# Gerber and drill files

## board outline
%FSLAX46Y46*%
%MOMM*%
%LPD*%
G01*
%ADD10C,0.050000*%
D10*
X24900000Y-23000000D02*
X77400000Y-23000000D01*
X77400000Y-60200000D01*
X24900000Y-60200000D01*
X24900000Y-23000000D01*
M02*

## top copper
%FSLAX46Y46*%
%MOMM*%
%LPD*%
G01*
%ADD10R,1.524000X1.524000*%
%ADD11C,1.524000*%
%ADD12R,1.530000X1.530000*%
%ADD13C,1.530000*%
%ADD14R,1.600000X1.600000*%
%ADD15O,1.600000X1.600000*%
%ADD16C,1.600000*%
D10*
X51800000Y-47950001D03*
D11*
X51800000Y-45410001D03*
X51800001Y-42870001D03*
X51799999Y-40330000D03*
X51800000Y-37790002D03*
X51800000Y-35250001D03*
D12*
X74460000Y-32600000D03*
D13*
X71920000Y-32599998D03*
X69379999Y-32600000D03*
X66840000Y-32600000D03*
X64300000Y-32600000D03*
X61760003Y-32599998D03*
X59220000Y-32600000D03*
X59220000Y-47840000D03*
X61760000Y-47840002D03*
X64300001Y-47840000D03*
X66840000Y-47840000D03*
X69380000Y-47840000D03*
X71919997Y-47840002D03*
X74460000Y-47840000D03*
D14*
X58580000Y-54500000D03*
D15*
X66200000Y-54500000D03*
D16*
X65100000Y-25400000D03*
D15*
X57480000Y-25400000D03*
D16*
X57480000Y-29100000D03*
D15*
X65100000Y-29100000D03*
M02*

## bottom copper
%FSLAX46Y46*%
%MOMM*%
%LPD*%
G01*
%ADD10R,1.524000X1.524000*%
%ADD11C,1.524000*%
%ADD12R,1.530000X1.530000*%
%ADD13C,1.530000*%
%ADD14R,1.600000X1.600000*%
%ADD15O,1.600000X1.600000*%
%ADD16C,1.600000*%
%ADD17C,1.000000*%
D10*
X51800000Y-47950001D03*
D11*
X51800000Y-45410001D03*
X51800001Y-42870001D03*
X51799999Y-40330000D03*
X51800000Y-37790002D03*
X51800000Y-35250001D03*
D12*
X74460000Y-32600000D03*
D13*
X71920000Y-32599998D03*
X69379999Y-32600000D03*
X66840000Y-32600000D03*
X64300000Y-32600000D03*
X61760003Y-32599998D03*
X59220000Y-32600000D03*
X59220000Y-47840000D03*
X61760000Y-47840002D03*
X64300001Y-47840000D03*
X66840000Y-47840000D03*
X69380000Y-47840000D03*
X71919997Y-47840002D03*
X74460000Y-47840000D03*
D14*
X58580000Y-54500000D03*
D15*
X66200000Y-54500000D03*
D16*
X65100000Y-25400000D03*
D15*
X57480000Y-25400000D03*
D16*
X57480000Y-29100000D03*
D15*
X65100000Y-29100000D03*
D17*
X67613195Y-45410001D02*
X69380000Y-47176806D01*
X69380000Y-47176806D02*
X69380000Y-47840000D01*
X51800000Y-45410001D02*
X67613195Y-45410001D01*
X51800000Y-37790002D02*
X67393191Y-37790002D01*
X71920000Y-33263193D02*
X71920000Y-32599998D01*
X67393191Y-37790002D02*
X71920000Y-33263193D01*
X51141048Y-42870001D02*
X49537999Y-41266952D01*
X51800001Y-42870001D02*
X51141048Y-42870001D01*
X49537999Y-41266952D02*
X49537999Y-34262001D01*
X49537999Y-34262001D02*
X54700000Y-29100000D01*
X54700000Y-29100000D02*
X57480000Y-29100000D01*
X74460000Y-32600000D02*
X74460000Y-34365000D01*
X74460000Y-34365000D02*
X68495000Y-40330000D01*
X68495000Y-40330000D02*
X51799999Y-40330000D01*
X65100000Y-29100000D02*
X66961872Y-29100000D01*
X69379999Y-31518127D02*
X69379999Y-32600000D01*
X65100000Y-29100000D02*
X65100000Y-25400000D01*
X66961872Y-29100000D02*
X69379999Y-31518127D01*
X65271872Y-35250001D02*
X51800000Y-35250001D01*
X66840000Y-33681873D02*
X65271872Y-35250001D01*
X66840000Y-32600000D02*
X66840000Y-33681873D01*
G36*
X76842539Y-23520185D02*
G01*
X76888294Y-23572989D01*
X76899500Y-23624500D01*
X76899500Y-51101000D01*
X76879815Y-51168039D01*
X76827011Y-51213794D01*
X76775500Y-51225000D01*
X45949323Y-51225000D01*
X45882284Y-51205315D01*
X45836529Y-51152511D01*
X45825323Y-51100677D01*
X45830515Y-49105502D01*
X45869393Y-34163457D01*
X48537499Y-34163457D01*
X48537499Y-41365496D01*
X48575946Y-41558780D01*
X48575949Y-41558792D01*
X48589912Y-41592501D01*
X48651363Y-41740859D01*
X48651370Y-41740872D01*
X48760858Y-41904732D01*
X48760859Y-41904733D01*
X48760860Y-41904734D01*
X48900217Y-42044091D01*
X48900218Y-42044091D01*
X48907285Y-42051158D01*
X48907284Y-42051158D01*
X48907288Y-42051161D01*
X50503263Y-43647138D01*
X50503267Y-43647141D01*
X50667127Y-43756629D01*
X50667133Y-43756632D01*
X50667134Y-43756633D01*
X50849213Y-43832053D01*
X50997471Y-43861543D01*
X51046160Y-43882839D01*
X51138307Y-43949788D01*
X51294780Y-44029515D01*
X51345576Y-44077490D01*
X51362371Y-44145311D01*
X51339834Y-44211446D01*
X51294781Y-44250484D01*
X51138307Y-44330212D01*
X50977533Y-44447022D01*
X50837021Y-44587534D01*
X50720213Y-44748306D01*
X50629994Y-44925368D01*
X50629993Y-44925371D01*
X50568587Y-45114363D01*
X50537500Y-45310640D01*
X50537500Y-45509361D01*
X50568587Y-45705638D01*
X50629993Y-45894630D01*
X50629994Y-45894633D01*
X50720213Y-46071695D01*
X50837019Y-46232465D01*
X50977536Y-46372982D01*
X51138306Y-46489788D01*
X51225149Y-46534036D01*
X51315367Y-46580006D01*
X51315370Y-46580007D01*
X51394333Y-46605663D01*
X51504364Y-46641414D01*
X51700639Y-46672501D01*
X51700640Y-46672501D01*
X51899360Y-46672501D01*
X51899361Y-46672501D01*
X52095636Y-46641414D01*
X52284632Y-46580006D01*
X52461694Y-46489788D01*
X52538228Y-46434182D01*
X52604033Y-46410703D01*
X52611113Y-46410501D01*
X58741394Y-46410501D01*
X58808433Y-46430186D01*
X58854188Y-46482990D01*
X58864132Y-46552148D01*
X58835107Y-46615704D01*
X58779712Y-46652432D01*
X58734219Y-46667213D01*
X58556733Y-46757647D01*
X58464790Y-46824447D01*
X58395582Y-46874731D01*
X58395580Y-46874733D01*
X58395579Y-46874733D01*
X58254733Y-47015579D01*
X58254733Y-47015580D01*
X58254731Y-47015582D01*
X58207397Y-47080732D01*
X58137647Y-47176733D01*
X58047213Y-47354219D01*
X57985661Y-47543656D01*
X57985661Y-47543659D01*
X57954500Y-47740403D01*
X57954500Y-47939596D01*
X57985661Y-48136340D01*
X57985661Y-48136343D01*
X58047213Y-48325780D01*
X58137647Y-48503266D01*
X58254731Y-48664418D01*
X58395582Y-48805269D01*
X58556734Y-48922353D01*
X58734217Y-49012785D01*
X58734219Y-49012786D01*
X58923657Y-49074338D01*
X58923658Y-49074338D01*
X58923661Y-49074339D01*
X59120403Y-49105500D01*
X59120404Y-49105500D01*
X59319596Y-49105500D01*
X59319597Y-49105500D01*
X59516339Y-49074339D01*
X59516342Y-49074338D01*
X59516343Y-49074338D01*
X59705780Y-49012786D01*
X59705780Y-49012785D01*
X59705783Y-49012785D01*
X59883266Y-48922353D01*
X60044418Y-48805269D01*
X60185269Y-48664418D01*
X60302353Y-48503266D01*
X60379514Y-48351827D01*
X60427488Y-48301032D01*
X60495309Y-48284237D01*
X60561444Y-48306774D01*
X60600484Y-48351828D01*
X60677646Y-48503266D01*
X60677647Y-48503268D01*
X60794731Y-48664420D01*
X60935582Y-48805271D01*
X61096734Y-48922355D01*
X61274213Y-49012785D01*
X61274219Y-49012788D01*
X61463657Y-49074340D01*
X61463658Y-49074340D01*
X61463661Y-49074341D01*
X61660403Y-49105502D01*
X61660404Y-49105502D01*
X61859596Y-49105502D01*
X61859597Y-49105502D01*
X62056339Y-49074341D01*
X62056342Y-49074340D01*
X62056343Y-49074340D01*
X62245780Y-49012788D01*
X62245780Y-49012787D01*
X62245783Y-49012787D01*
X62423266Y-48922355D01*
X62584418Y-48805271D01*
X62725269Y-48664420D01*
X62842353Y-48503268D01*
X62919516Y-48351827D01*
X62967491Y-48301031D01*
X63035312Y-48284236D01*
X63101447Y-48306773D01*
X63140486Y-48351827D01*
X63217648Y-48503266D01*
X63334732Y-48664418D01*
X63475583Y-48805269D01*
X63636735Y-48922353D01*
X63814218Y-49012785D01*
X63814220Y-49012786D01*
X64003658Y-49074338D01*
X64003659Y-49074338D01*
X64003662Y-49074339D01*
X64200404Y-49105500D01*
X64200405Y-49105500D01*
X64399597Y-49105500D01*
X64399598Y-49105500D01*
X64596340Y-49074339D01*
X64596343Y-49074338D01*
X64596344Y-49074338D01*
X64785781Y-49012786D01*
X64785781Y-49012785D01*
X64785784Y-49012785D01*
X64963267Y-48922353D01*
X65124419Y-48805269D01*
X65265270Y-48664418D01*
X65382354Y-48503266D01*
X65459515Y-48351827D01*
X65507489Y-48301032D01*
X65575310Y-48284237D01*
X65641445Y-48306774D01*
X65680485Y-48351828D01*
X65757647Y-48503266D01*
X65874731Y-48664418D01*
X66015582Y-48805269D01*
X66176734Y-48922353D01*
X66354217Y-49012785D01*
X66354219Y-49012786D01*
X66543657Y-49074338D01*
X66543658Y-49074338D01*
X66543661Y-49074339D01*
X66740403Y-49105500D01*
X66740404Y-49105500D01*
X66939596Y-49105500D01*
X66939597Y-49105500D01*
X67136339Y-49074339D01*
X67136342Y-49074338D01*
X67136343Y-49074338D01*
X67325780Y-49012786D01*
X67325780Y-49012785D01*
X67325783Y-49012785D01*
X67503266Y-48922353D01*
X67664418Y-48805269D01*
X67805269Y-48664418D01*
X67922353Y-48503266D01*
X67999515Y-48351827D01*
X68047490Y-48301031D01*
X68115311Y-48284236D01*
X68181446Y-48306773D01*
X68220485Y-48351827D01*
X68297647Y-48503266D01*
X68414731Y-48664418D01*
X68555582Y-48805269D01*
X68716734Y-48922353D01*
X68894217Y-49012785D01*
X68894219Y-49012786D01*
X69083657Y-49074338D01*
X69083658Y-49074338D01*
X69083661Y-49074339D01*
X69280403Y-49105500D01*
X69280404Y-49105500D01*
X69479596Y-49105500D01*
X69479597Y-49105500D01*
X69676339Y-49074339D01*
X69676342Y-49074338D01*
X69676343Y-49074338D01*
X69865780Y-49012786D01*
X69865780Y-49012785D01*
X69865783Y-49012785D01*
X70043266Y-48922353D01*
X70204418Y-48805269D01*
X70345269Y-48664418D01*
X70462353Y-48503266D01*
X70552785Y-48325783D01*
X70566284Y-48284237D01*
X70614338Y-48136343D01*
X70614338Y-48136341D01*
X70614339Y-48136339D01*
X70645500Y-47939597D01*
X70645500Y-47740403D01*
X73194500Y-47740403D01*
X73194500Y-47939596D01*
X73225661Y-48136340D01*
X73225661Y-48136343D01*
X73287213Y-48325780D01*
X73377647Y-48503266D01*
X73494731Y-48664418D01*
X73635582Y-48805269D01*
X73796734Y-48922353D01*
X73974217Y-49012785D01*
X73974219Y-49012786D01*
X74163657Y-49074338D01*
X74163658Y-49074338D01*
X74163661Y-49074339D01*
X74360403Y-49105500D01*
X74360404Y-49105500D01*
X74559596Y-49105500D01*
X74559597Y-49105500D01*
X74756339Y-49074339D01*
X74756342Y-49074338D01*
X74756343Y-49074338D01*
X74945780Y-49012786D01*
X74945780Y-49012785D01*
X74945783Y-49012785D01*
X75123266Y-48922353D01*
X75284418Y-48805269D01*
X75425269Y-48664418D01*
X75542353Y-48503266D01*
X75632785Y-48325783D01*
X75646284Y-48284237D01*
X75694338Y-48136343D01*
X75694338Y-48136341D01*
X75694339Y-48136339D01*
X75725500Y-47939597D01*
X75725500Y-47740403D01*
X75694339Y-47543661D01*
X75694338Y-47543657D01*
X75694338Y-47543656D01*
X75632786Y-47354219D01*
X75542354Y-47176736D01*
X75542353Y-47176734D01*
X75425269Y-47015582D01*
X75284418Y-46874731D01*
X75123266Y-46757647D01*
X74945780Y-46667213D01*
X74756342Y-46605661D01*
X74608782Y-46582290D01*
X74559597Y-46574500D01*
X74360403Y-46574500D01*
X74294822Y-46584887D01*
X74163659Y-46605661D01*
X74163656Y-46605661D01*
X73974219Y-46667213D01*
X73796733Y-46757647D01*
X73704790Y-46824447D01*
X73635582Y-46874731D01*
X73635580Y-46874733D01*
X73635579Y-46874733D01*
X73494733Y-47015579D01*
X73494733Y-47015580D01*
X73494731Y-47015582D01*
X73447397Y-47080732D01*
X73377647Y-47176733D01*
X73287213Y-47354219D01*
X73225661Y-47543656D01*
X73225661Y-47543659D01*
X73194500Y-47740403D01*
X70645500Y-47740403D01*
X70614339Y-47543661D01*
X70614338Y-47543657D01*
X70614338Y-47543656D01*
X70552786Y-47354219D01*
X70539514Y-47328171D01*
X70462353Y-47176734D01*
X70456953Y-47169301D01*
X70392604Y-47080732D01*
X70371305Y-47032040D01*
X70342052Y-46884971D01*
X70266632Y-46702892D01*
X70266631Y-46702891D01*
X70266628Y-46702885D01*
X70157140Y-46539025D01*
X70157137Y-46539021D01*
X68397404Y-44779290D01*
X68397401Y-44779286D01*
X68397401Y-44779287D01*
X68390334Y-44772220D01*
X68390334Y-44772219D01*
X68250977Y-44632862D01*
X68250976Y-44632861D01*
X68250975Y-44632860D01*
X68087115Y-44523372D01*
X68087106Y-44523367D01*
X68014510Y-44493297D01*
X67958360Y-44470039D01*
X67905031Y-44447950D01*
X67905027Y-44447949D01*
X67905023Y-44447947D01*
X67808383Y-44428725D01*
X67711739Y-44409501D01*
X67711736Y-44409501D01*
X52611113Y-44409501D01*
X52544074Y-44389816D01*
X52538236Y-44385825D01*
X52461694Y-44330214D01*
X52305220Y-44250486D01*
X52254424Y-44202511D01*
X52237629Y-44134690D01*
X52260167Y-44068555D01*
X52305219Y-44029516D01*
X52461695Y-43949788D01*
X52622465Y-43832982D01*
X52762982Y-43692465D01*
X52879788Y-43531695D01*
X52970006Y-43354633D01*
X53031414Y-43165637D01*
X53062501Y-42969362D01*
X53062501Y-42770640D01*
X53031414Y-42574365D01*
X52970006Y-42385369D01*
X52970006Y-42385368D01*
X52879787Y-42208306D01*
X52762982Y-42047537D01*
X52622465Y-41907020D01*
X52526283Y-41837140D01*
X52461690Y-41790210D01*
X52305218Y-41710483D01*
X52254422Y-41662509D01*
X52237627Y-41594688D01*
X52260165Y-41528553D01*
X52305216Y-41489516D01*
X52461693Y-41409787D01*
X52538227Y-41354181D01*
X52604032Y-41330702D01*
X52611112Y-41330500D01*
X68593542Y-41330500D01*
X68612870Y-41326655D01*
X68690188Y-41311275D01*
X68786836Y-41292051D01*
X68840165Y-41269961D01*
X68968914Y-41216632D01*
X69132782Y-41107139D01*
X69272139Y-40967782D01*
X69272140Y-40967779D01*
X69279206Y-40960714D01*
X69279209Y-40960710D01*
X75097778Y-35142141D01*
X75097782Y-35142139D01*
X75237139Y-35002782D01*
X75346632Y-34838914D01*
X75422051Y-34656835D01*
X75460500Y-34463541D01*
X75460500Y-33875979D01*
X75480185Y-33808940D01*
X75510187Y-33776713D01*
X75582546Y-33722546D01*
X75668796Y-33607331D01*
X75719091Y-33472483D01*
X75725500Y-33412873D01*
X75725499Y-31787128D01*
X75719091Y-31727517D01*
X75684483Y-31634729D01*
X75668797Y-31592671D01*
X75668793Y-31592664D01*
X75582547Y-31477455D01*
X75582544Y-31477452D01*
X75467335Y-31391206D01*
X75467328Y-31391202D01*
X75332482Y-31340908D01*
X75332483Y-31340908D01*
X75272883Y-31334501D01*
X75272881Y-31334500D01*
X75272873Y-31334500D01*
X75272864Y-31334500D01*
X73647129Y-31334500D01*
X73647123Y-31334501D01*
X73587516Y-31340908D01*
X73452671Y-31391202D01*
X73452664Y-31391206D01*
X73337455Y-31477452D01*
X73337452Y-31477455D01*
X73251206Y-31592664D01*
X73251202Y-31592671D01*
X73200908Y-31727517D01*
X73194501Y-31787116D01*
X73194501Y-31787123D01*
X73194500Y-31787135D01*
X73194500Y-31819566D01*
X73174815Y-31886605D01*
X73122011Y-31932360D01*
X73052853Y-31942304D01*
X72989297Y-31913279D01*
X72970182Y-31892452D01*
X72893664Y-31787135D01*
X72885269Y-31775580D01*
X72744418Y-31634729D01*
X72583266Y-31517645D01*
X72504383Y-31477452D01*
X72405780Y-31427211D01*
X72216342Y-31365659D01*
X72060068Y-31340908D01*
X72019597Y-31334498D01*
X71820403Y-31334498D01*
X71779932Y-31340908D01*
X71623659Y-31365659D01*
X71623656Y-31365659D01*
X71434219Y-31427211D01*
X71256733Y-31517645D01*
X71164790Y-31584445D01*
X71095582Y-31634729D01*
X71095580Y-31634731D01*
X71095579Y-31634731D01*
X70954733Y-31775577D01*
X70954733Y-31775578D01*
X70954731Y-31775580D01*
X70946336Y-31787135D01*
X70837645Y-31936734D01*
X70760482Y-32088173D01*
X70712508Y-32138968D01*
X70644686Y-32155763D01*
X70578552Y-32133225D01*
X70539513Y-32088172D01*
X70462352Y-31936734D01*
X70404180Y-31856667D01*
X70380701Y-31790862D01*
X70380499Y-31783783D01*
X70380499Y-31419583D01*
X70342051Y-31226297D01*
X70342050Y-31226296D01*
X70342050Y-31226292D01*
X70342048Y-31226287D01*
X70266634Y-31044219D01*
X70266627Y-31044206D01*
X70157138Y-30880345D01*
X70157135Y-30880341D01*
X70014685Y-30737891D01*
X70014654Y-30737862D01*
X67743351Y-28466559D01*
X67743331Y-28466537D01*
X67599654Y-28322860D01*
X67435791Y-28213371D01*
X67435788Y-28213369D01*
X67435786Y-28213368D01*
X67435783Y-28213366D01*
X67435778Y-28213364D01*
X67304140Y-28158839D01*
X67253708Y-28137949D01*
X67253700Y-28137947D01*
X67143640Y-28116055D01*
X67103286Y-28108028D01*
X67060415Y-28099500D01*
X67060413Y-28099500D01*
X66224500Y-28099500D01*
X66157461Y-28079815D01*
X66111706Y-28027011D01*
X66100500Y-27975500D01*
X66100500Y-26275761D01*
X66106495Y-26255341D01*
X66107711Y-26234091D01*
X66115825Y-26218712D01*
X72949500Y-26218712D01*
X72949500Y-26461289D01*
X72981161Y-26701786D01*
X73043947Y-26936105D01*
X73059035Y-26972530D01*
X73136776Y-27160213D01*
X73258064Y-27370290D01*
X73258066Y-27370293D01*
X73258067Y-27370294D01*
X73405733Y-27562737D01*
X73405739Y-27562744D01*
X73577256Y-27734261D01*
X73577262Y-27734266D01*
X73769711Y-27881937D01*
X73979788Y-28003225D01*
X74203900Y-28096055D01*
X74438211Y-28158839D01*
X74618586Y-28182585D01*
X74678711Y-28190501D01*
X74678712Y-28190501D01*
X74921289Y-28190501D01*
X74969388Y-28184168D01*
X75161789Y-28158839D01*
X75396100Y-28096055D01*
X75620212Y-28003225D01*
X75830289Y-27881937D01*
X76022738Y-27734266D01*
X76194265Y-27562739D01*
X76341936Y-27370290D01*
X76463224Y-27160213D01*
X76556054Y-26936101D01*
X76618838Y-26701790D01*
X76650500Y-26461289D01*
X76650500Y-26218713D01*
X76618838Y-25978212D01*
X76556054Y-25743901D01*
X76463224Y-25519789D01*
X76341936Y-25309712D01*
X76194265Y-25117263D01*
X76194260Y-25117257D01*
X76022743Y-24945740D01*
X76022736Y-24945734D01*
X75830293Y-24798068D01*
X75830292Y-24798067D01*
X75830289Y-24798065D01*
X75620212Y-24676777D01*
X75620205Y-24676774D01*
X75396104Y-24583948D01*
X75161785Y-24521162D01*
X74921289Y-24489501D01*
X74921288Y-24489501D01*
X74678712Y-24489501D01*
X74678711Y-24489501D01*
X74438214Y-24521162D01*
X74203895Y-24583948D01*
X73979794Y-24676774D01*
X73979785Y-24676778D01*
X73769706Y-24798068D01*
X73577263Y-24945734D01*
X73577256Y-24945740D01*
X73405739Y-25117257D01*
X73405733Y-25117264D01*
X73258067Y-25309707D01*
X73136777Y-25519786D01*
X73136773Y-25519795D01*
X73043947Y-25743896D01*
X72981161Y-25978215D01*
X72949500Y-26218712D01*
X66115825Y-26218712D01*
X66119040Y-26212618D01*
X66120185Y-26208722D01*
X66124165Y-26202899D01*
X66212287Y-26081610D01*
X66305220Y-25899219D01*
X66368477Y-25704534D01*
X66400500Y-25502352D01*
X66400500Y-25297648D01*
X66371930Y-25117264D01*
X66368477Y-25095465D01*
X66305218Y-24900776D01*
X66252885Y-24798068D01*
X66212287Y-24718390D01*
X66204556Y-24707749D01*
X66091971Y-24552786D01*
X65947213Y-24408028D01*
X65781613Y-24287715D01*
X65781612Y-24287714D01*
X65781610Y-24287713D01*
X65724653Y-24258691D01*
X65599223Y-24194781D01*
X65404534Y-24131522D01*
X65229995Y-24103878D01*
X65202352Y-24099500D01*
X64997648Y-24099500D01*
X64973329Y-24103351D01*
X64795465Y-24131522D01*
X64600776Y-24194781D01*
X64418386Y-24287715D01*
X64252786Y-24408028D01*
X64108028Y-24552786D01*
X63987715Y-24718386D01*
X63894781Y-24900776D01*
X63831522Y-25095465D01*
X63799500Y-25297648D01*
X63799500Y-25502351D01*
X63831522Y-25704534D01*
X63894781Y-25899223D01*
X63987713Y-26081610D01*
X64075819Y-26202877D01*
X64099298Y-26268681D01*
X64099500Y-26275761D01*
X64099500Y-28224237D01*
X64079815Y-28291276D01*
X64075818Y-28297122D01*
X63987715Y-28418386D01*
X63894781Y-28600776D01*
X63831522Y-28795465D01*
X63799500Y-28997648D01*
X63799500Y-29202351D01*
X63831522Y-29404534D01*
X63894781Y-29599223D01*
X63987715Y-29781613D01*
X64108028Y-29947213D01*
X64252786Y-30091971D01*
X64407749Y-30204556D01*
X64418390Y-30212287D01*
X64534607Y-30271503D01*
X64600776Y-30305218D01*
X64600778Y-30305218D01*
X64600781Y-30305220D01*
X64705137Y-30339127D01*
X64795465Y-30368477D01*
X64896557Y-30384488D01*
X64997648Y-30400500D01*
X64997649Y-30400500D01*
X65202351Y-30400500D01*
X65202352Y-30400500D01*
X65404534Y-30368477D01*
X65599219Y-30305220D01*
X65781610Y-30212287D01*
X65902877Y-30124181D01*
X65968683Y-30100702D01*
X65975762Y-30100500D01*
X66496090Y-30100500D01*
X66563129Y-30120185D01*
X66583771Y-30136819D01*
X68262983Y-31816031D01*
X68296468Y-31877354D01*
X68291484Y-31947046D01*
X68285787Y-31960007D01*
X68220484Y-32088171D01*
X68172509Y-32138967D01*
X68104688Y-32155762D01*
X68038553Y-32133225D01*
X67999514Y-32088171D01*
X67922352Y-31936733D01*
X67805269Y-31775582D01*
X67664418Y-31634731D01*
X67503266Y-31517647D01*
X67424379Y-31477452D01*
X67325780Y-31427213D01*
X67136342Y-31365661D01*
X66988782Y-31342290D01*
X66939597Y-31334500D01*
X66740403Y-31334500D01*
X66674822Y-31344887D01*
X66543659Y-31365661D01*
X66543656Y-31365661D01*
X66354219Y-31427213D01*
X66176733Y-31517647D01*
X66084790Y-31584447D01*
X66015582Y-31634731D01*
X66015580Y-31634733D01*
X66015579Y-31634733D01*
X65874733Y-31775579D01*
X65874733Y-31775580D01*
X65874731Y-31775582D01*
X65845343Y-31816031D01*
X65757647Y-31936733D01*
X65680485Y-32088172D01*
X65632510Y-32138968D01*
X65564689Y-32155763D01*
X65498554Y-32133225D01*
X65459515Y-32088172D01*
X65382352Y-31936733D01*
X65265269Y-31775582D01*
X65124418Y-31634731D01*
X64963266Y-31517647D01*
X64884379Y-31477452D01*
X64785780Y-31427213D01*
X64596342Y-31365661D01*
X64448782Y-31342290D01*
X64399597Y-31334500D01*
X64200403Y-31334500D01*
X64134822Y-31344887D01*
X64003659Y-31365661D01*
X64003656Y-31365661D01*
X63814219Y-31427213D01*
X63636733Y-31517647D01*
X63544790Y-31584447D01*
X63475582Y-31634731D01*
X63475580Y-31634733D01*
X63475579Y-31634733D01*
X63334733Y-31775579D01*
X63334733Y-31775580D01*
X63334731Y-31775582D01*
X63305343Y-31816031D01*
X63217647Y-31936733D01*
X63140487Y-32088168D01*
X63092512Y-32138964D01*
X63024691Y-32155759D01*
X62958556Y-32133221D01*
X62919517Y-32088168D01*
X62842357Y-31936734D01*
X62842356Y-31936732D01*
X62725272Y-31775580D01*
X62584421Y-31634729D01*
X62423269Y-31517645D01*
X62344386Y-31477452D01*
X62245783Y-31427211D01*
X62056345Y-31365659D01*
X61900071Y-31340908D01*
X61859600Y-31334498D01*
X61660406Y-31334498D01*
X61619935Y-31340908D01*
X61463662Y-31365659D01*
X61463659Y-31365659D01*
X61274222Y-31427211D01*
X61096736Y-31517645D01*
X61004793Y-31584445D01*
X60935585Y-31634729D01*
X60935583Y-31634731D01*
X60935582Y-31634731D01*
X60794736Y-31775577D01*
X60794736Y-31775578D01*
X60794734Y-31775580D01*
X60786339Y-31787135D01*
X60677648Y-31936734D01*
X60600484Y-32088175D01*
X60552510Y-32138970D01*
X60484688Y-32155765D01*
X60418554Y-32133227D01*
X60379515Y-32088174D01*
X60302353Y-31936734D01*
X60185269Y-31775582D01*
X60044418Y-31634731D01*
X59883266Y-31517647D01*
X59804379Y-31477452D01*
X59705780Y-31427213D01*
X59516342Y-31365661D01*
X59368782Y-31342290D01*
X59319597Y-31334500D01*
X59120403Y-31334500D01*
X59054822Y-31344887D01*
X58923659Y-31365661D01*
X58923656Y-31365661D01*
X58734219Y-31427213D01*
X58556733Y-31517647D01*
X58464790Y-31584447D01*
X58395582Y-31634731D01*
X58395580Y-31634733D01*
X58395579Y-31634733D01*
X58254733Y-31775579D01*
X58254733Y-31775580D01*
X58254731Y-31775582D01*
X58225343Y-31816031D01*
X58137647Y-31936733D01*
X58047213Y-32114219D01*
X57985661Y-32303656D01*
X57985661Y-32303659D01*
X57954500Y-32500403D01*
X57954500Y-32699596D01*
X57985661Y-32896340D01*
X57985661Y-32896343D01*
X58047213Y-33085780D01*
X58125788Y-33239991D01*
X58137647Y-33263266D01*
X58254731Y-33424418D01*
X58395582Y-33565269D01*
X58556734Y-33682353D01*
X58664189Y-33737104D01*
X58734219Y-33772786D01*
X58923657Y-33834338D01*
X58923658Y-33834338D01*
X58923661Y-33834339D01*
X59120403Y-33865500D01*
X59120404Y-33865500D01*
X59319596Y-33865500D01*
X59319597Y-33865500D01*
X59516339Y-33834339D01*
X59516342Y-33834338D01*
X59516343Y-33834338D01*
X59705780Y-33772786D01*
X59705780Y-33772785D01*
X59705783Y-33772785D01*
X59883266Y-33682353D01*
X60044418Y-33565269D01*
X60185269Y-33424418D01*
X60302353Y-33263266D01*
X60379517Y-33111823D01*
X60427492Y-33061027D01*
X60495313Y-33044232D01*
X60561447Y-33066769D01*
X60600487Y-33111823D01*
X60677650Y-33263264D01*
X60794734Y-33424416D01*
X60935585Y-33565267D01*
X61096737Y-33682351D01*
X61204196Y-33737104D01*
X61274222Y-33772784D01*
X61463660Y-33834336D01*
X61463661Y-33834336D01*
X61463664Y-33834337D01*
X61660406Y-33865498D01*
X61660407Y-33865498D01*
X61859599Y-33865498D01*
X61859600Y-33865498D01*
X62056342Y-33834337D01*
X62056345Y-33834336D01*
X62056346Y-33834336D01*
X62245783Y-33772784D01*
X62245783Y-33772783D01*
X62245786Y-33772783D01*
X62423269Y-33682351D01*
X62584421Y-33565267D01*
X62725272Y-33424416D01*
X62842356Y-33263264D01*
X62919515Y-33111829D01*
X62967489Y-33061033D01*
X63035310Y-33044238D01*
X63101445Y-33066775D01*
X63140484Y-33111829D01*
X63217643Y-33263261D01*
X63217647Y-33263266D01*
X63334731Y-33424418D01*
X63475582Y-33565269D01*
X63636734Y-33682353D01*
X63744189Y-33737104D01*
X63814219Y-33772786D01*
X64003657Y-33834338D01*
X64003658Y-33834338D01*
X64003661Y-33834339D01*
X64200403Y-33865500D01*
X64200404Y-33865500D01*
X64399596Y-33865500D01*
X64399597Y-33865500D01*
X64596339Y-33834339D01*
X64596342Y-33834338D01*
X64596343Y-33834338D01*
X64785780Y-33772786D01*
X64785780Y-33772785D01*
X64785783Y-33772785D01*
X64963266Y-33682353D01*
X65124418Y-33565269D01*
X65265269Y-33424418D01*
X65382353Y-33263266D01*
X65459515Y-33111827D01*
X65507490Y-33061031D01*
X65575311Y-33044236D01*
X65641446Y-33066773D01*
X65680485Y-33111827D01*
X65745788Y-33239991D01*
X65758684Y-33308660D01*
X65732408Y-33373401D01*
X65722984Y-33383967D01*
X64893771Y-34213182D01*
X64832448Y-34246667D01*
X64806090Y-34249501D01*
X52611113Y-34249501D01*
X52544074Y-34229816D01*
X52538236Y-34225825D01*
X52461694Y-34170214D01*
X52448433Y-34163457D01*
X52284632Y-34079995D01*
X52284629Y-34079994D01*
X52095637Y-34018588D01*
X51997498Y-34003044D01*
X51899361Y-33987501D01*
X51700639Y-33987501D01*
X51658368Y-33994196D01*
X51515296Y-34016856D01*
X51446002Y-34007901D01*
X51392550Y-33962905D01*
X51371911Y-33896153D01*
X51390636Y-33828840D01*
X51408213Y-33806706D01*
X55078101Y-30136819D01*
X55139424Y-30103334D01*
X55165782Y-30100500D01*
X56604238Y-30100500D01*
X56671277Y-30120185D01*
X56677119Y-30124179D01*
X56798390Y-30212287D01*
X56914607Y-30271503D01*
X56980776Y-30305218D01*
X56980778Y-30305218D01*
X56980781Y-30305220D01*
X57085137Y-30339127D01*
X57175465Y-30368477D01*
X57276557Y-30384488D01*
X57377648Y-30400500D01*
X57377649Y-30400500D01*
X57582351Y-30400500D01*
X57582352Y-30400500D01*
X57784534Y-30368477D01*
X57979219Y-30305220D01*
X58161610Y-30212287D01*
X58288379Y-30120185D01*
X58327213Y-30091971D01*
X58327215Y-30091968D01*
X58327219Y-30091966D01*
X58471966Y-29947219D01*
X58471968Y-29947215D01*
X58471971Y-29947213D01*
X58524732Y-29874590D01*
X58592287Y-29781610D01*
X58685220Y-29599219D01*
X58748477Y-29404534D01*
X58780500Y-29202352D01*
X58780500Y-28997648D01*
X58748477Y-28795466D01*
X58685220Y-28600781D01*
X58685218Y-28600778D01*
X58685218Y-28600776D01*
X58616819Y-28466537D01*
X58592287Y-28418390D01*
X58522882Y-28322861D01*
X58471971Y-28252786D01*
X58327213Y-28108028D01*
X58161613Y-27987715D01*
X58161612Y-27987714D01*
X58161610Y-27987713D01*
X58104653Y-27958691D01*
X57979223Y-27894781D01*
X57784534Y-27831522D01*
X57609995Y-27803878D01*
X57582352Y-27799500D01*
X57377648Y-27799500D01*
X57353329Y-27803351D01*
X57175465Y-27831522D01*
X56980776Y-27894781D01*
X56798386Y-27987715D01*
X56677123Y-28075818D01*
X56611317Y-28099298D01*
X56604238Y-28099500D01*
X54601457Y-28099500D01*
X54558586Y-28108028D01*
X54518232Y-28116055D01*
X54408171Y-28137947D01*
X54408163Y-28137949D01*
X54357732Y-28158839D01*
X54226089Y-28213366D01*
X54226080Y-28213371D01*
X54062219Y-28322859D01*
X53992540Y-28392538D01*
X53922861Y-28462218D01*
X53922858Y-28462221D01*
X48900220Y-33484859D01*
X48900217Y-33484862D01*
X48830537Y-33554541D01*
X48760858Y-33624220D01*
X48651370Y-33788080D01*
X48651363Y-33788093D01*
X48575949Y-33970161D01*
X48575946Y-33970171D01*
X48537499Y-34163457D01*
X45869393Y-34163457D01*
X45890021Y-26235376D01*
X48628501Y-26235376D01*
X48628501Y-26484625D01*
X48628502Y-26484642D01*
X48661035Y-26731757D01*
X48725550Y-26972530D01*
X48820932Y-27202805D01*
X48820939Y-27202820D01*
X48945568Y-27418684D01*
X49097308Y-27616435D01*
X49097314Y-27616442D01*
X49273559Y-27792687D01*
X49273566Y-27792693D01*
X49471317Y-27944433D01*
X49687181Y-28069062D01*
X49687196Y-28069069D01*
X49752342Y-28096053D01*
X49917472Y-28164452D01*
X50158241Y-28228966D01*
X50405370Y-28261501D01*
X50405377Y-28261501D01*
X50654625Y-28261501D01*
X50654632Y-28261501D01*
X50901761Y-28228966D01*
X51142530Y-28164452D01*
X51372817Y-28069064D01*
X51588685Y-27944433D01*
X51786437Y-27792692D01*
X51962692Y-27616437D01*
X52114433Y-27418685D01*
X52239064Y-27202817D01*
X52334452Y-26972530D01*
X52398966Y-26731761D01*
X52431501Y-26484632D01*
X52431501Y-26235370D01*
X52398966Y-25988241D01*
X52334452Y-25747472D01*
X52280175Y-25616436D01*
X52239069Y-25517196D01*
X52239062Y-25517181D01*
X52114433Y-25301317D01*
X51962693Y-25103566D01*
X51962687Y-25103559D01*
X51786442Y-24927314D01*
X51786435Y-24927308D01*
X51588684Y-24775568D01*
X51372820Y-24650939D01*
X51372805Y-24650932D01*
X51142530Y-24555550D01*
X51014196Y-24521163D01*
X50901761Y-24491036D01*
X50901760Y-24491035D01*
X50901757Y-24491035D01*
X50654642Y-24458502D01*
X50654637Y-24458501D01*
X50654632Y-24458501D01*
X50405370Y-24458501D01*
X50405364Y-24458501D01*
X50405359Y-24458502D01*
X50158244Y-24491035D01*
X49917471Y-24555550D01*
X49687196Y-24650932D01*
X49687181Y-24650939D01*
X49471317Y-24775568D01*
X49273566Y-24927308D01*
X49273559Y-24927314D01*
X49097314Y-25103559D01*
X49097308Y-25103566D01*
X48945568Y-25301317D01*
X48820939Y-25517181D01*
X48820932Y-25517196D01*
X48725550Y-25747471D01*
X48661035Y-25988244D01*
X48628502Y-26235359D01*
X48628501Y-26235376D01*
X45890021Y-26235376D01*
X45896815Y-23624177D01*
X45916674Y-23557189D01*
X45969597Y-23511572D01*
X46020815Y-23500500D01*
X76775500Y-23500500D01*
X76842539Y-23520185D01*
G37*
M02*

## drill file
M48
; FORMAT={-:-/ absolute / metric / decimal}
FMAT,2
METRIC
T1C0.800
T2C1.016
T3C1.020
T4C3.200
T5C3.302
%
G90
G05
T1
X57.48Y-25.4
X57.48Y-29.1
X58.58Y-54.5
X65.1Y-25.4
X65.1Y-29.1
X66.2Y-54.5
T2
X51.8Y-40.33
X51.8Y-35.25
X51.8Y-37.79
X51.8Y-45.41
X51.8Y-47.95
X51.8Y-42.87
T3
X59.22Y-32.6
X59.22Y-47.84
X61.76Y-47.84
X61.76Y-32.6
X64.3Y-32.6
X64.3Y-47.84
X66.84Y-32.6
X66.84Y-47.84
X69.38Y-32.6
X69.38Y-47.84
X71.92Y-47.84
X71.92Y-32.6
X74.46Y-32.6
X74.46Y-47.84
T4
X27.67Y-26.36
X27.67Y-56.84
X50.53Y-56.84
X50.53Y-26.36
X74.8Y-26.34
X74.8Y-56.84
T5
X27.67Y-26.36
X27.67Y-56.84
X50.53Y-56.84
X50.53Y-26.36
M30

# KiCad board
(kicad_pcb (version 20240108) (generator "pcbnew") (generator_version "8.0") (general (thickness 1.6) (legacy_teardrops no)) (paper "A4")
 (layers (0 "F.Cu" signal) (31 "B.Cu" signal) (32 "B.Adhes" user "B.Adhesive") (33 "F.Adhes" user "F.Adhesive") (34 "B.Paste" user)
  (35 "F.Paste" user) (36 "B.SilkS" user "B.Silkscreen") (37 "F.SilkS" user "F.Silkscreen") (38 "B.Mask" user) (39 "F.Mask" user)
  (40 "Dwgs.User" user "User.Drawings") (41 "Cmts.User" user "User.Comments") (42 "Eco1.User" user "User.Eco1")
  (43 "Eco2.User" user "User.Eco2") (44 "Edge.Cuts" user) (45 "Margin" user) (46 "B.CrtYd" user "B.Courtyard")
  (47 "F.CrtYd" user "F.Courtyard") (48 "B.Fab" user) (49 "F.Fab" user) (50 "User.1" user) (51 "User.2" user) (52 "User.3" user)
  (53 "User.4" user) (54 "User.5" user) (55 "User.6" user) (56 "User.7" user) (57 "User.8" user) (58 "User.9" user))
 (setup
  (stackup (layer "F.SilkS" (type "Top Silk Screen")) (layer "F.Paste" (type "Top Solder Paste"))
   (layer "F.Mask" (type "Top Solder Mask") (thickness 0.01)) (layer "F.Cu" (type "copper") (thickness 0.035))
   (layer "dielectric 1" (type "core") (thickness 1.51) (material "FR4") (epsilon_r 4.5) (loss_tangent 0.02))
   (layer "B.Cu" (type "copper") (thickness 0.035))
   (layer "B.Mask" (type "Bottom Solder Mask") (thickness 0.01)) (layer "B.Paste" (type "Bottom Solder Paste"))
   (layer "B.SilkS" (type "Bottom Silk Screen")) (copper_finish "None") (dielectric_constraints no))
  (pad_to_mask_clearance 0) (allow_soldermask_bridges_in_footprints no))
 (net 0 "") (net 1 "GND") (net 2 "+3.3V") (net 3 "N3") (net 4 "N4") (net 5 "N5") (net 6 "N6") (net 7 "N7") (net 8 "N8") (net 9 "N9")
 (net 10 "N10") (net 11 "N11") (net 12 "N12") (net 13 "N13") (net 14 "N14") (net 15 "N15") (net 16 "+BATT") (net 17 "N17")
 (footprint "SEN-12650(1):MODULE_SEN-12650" (layer "F.Cu") (at 53.07 59.380001 90)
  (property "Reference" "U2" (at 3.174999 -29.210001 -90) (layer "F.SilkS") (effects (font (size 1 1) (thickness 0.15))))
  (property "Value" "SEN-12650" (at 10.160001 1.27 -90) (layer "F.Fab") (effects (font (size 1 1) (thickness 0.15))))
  (pad "" np_thru_hole circle (at 2.54 -25.399998 90) (size 3.302 3.302) (drill 3.302) (layers "*.Cu" "*.Mask"))
  (pad "" np_thru_hole circle (at 2.54 -2.54 90) (size 3.302 3.302) (drill 3.302) (layers "*.Cu" "*.Mask"))
  (pad "" np_thru_hole circle (at 33.02 -25.4 90) (size 3.302 3.302) (drill 3.302) (layers "*.Cu" "*.Mask"))
  (pad "" np_thru_hole circle (at 33.02 -2.539999 90) (size 3.302 3.302) (drill 3.302) (layers "*.Cu" "*.Mask"))
  (pad "JP3_1" thru_hole rect (at 11.43 -1.27 90) (size 1.524 1.524) (drill 1.016) (layers "*.Cu" "*.Mask") (remove_unused_layers no)
   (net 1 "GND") (solder_mask_margin 0.102))
  (pad "JP3_2" thru_hole circle (at 13.97 -1.27 90) (size 1.524 1.524) (drill 1.016) (layers "*.Cu" "*.Mask") (remove_unused_layers no)
   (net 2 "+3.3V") (solder_mask_margin 0.102))
  (pad "JP3_3" thru_hole circle (at 16.51 -1.269999 90) (size 1.524 1.524) (drill 1.016) (layers "*.Cu" "*.Mask") (remove_unused_layers no)
   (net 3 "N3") (solder_mask_margin 0.102))
  (pad "JP3_4" thru_hole circle (at 19.050001 -1.270001 90) (size 1.524 1.524) (drill 1.016) (layers "*.Cu" "*.Mask")
   (remove_unused_layers no) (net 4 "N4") (solder_mask_margin 0.102))
  (pad "JP3_5" thru_hole circle (at 21.589999 -1.27 90) (size 1.524 1.524) (drill 1.016) (layers "*.Cu" "*.Mask") (remove_unused_layers no)
   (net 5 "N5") (solder_mask_margin 0.102))
  (pad "JP3_6" thru_hole circle (at 24.13 -1.27 90) (size 1.524 1.524) (drill 1.016) (layers "*.Cu" "*.Mask") (remove_unused_layers no)
   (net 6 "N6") (solder_mask_margin 0.102)))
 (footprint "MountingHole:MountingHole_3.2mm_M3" (layer "F.Cu") (at 74.8 26.340001)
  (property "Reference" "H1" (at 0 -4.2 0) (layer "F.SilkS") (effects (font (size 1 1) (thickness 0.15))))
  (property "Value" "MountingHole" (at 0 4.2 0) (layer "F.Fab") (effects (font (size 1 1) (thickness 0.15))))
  (pad "" np_thru_hole circle (at 0 0) (size 3.2 3.2) (drill 3.2) (layers "*.Cu" "*.Mask")))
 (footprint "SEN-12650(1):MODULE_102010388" (layer "F.Cu") (at 66.84 40.22 -90)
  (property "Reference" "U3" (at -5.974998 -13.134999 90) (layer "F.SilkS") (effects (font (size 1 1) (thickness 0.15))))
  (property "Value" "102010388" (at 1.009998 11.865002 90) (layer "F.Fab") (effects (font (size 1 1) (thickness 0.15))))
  (pad "1" thru_hole rect (at -7.62 -7.62 270) (size 1.53 1.53) (drill 1.02) (layers "*.Cu" "*.Mask") (remove_unused_layers no) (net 4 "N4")
   (solder_mask_margin 0.102))
  (pad "2" thru_hole circle (at -7.620002 -5.08 270) (size 1.53 1.53) (drill 1.02) (layers "*.Cu" "*.Mask") (remove_unused_layers no)
   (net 5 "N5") (solder_mask_margin 0.102))
  (pad "3" thru_hole circle (at -7.62 -2.539999 270) (size 1.53 1.53) (drill 1.02) (layers "*.Cu" "*.Mask") (remove_unused_layers no)
   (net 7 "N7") (solder_mask_margin 0.102))
  (pad "4" thru_hole circle (at -7.62 0 270) (size 1.53 1.53) (drill 1.02) (layers "*.Cu" "*.Mask") (remove_unused_layers no) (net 6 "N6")
   (solder_mask_margin 0.102))
  (pad "5" thru_hole circle (at -7.62 2.54 270) (size 1.53 1.53) (drill 1.02) (layers "*.Cu" "*.Mask") (remove_unused_layers no)
   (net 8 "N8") (solder_mask_margin 0.102))
  (pad "6" thru_hole circle (at -7.620002 5.079997 270) (size 1.53 1.53) (drill 1.02) (layers "*.Cu" "*.Mask") (remove_unused_layers no)
   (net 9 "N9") (solder_mask_margin 0.102))
  (pad "7" thru_hole circle (at -7.62 7.62 270) (size 1.53 1.53) (drill 1.02) (layers "*.Cu" "*.Mask") (remove_unused_layers no)
   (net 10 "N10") (solder_mask_margin 0.102))
  (pad "8" thru_hole circle (at 7.62 7.62 270) (size 1.53 1.53) (drill 1.02) (layers "*.Cu" "*.Mask") (remove_unused_layers no)
   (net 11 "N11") (solder_mask_margin 0.102))
  (pad "9" thru_hole circle (at 7.620002 5.08 270) (size 1.53 1.53) (drill 1.02) (layers "*.Cu" "*.Mask") (remove_unused_layers no)
   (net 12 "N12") (solder_mask_margin 0.102))
  (pad "10" thru_hole circle (at 7.62 2.539999 270) (size 1.53 1.53) (drill 1.02) (layers "*.Cu" "*.Mask") (remove_unused_layers no)
   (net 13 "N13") (solder_mask_margin 0.102))
  (pad "11" thru_hole circle (at 7.62 0 270) (size 1.53 1.53) (drill 1.02) (layers "*.Cu" "*.Mask") (remove_unused_layers no) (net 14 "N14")
   (solder_mask_margin 0.102))
  (pad "12" thru_hole circle (at 7.62 -2.54 270) (size 1.53 1.53) (drill 1.02) (layers "*.Cu" "*.Mask") (remove_unused_layers no)
   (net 2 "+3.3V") (solder_mask_margin 0.102))
  (pad "13" thru_hole circle (at 7.620002 -5.079997 270) (size 1.53 1.53) (drill 1.02) (layers "*.Cu" "*.Mask") (remove_unused_layers no)
   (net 1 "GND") (solder_mask_margin 0.102))
  (pad "14" thru_hole circle (at 7.62 -7.62 270) (size 1.53 1.53) (drill 1.02) (layers "*.Cu" "*.Mask") (remove_unused_layers no)
   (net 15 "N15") (solder_mask_margin 0.102)))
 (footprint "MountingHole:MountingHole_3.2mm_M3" (layer "F.Cu") (at 27.67 26.360001)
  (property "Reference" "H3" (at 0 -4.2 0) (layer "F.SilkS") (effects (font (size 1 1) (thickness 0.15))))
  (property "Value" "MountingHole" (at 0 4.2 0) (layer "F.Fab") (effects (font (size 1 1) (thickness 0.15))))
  (pad "" np_thru_hole circle (at 0 0) (size 3.2 3.2) (drill 3.2) (layers "*.Cu" "*.Mask")))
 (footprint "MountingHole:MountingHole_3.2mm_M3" (layer "F.Cu") (at 74.8 56.840001)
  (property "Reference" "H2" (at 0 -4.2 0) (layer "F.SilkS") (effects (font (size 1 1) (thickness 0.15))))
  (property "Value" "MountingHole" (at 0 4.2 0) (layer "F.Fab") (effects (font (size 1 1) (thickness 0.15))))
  (pad "" np_thru_hole circle (at 0 0) (size 3.2 3.2) (drill 3.2) (layers "*.Cu" "*.Mask")))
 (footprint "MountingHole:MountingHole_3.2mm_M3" (layer "F.Cu") (at 27.670002 56.840001)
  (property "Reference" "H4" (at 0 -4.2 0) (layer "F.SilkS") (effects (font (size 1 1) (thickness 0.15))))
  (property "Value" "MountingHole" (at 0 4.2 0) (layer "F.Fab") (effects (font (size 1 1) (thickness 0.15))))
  (pad "" np_thru_hole circle (at 0 0) (size 3.2 3.2) (drill 3.2) (layers "*.Cu" "*.Mask")))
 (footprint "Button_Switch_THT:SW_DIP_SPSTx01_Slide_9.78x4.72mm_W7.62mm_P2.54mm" (layer "F.Cu") (at 58.58 54.5)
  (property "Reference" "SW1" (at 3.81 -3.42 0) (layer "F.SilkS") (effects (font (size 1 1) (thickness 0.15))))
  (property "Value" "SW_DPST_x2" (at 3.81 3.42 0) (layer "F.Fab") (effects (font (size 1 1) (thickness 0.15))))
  (pad "1" thru_hole rect (at 0 0) (size 1.6 1.6) (drill 0.8) (layers "*.Cu" "*.Mask") (remove_unused_layers no) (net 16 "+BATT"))
  (pad "2" thru_hole oval (at 7.62 0) (size 1.6 1.6) (drill 0.8) (layers "*.Cu" "*.Mask") (remove_unused_layers no) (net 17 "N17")))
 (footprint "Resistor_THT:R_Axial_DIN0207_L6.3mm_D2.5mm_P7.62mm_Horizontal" (layer "F.Cu") (at 65.1 25.4 180)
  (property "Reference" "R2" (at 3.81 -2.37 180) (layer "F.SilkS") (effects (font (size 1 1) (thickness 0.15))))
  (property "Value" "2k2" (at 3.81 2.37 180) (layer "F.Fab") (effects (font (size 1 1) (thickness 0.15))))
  (pad "1" thru_hole circle (at 0 0 180) (size 1.6 1.6) (drill 0.8) (layers "*.Cu" "*.Mask") (remove_unused_layers no) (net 7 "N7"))
  (pad "2" thru_hole oval (at 7.62 0 180) (size 1.6 1.6) (drill 0.8) (layers "*.Cu" "*.Mask") (remove_unused_layers no) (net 1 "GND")))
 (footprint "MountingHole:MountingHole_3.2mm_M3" (layer "F.Cu") (at 50.53 56.840001)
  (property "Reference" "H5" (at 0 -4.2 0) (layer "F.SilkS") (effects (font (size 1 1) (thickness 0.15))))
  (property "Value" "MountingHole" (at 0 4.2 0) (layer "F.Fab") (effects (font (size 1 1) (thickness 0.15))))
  (pad "" np_thru_hole circle (at 0 0) (size 3.2 3.2) (drill 3.2) (layers "*.Cu" "*.Mask")))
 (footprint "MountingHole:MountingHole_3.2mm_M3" (layer "F.Cu") (at 50.530001 26.360001)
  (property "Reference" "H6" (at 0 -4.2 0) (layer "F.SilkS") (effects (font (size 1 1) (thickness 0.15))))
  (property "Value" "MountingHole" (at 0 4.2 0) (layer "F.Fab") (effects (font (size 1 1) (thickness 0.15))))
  (pad "" np_thru_hole circle (at 0 0) (size 3.2 3.2) (drill 3.2) (layers "*.Cu" "*.Mask")))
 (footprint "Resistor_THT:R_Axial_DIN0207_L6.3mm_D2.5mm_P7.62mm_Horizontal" (layer "F.Cu") (at 57.48 29.1)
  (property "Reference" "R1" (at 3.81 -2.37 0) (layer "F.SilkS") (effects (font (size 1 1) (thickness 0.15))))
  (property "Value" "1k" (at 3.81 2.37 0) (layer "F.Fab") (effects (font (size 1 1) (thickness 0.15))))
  (pad "1" thru_hole circle (at 0 0) (size 1.6 1.6) (drill 0.8) (layers "*.Cu" "*.Mask") (remove_unused_layers no) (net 3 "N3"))
  (pad "2" thru_hole oval (at 7.62 0) (size 1.6 1.6) (drill 0.8) (layers "*.Cu" "*.Mask") (remove_unused_layers no) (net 7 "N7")))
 (gr_rect (start 24.9 23) (end 77.4 60.2) (stroke (width 0.05) (type default)) (fill none) (layer "Edge.Cuts"))
 (segment (start 67.613195 45.410001) (end 69.38 47.176806) (width 1) (layer "B.Cu") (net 2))
 (segment (start 69.38 47.176806) (end 69.38 47.84) (width 1) (layer "B.Cu") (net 2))
 (segment (start 51.8 45.410001) (end 67.613195 45.410001) (width 1) (layer "B.Cu") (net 2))
 (segment (start 51.8 37.790002) (end 67.393191 37.790002) (width 1) (layer "B.Cu") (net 5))
 (segment (start 71.92 33.263193) (end 71.92 32.599998) (width 1) (layer "B.Cu") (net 5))
 (segment (start 67.393191 37.790002) (end 71.92 33.263193) (width 1) (layer "B.Cu") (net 5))
 (segment (start 51.141048 42.870001) (end 49.537999 41.266952) (width 1) (layer "B.Cu") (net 3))
 (segment (start 51.800001 42.870001) (end 51.141048 42.870001) (width 1) (layer "B.Cu") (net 3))
 (segment (start 49.537999 41.266952) (end 49.537999 34.262001) (width 1) (layer "B.Cu") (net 3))
 (segment (start 49.537999 34.262001) (end 54.7 29.1) (width 1) (layer "B.Cu") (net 3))
 (segment (start 54.7 29.1) (end 57.48 29.1) (width 1) (layer "B.Cu") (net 3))
 (segment (start 74.46 32.6) (end 74.46 34.365) (width 1) (layer "B.Cu") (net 4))
 (segment (start 74.46 34.365) (end 68.495 40.33) (width 1) (layer "B.Cu") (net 4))
 (segment (start 68.495 40.33) (end 51.799999 40.33) (width 1) (layer "B.Cu") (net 4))
 (segment (start 65.1 29.1) (end 66.961872 29.1) (width 1) (layer "B.Cu") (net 7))
 (segment (start 69.379999 31.518127) (end 69.379999 32.6) (width 1) (layer "B.Cu") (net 7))
 (segment (start 65.1 29.1) (end 65.1 25.4) (width 1) (layer "B.Cu") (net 7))
 (segment (start 66.961872 29.1) (end 69.379999 31.518127) (width 1) (layer "B.Cu") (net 7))
 (segment (start 65.271872 35.250001) (end 51.8 35.250001) (width 1) (layer "B.Cu") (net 6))
 (segment (start 66.84 33.681873) (end 65.271872 35.250001) (width 1) (layer "B.Cu") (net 6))
 (segment (start 66.84 32.6) (end 66.84 33.681873) (width 1) (layer "B.Cu") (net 6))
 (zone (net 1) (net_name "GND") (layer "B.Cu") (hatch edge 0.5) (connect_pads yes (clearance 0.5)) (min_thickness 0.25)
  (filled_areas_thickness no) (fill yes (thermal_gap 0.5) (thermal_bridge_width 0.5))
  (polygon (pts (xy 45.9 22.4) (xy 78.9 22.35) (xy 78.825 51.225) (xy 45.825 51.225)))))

